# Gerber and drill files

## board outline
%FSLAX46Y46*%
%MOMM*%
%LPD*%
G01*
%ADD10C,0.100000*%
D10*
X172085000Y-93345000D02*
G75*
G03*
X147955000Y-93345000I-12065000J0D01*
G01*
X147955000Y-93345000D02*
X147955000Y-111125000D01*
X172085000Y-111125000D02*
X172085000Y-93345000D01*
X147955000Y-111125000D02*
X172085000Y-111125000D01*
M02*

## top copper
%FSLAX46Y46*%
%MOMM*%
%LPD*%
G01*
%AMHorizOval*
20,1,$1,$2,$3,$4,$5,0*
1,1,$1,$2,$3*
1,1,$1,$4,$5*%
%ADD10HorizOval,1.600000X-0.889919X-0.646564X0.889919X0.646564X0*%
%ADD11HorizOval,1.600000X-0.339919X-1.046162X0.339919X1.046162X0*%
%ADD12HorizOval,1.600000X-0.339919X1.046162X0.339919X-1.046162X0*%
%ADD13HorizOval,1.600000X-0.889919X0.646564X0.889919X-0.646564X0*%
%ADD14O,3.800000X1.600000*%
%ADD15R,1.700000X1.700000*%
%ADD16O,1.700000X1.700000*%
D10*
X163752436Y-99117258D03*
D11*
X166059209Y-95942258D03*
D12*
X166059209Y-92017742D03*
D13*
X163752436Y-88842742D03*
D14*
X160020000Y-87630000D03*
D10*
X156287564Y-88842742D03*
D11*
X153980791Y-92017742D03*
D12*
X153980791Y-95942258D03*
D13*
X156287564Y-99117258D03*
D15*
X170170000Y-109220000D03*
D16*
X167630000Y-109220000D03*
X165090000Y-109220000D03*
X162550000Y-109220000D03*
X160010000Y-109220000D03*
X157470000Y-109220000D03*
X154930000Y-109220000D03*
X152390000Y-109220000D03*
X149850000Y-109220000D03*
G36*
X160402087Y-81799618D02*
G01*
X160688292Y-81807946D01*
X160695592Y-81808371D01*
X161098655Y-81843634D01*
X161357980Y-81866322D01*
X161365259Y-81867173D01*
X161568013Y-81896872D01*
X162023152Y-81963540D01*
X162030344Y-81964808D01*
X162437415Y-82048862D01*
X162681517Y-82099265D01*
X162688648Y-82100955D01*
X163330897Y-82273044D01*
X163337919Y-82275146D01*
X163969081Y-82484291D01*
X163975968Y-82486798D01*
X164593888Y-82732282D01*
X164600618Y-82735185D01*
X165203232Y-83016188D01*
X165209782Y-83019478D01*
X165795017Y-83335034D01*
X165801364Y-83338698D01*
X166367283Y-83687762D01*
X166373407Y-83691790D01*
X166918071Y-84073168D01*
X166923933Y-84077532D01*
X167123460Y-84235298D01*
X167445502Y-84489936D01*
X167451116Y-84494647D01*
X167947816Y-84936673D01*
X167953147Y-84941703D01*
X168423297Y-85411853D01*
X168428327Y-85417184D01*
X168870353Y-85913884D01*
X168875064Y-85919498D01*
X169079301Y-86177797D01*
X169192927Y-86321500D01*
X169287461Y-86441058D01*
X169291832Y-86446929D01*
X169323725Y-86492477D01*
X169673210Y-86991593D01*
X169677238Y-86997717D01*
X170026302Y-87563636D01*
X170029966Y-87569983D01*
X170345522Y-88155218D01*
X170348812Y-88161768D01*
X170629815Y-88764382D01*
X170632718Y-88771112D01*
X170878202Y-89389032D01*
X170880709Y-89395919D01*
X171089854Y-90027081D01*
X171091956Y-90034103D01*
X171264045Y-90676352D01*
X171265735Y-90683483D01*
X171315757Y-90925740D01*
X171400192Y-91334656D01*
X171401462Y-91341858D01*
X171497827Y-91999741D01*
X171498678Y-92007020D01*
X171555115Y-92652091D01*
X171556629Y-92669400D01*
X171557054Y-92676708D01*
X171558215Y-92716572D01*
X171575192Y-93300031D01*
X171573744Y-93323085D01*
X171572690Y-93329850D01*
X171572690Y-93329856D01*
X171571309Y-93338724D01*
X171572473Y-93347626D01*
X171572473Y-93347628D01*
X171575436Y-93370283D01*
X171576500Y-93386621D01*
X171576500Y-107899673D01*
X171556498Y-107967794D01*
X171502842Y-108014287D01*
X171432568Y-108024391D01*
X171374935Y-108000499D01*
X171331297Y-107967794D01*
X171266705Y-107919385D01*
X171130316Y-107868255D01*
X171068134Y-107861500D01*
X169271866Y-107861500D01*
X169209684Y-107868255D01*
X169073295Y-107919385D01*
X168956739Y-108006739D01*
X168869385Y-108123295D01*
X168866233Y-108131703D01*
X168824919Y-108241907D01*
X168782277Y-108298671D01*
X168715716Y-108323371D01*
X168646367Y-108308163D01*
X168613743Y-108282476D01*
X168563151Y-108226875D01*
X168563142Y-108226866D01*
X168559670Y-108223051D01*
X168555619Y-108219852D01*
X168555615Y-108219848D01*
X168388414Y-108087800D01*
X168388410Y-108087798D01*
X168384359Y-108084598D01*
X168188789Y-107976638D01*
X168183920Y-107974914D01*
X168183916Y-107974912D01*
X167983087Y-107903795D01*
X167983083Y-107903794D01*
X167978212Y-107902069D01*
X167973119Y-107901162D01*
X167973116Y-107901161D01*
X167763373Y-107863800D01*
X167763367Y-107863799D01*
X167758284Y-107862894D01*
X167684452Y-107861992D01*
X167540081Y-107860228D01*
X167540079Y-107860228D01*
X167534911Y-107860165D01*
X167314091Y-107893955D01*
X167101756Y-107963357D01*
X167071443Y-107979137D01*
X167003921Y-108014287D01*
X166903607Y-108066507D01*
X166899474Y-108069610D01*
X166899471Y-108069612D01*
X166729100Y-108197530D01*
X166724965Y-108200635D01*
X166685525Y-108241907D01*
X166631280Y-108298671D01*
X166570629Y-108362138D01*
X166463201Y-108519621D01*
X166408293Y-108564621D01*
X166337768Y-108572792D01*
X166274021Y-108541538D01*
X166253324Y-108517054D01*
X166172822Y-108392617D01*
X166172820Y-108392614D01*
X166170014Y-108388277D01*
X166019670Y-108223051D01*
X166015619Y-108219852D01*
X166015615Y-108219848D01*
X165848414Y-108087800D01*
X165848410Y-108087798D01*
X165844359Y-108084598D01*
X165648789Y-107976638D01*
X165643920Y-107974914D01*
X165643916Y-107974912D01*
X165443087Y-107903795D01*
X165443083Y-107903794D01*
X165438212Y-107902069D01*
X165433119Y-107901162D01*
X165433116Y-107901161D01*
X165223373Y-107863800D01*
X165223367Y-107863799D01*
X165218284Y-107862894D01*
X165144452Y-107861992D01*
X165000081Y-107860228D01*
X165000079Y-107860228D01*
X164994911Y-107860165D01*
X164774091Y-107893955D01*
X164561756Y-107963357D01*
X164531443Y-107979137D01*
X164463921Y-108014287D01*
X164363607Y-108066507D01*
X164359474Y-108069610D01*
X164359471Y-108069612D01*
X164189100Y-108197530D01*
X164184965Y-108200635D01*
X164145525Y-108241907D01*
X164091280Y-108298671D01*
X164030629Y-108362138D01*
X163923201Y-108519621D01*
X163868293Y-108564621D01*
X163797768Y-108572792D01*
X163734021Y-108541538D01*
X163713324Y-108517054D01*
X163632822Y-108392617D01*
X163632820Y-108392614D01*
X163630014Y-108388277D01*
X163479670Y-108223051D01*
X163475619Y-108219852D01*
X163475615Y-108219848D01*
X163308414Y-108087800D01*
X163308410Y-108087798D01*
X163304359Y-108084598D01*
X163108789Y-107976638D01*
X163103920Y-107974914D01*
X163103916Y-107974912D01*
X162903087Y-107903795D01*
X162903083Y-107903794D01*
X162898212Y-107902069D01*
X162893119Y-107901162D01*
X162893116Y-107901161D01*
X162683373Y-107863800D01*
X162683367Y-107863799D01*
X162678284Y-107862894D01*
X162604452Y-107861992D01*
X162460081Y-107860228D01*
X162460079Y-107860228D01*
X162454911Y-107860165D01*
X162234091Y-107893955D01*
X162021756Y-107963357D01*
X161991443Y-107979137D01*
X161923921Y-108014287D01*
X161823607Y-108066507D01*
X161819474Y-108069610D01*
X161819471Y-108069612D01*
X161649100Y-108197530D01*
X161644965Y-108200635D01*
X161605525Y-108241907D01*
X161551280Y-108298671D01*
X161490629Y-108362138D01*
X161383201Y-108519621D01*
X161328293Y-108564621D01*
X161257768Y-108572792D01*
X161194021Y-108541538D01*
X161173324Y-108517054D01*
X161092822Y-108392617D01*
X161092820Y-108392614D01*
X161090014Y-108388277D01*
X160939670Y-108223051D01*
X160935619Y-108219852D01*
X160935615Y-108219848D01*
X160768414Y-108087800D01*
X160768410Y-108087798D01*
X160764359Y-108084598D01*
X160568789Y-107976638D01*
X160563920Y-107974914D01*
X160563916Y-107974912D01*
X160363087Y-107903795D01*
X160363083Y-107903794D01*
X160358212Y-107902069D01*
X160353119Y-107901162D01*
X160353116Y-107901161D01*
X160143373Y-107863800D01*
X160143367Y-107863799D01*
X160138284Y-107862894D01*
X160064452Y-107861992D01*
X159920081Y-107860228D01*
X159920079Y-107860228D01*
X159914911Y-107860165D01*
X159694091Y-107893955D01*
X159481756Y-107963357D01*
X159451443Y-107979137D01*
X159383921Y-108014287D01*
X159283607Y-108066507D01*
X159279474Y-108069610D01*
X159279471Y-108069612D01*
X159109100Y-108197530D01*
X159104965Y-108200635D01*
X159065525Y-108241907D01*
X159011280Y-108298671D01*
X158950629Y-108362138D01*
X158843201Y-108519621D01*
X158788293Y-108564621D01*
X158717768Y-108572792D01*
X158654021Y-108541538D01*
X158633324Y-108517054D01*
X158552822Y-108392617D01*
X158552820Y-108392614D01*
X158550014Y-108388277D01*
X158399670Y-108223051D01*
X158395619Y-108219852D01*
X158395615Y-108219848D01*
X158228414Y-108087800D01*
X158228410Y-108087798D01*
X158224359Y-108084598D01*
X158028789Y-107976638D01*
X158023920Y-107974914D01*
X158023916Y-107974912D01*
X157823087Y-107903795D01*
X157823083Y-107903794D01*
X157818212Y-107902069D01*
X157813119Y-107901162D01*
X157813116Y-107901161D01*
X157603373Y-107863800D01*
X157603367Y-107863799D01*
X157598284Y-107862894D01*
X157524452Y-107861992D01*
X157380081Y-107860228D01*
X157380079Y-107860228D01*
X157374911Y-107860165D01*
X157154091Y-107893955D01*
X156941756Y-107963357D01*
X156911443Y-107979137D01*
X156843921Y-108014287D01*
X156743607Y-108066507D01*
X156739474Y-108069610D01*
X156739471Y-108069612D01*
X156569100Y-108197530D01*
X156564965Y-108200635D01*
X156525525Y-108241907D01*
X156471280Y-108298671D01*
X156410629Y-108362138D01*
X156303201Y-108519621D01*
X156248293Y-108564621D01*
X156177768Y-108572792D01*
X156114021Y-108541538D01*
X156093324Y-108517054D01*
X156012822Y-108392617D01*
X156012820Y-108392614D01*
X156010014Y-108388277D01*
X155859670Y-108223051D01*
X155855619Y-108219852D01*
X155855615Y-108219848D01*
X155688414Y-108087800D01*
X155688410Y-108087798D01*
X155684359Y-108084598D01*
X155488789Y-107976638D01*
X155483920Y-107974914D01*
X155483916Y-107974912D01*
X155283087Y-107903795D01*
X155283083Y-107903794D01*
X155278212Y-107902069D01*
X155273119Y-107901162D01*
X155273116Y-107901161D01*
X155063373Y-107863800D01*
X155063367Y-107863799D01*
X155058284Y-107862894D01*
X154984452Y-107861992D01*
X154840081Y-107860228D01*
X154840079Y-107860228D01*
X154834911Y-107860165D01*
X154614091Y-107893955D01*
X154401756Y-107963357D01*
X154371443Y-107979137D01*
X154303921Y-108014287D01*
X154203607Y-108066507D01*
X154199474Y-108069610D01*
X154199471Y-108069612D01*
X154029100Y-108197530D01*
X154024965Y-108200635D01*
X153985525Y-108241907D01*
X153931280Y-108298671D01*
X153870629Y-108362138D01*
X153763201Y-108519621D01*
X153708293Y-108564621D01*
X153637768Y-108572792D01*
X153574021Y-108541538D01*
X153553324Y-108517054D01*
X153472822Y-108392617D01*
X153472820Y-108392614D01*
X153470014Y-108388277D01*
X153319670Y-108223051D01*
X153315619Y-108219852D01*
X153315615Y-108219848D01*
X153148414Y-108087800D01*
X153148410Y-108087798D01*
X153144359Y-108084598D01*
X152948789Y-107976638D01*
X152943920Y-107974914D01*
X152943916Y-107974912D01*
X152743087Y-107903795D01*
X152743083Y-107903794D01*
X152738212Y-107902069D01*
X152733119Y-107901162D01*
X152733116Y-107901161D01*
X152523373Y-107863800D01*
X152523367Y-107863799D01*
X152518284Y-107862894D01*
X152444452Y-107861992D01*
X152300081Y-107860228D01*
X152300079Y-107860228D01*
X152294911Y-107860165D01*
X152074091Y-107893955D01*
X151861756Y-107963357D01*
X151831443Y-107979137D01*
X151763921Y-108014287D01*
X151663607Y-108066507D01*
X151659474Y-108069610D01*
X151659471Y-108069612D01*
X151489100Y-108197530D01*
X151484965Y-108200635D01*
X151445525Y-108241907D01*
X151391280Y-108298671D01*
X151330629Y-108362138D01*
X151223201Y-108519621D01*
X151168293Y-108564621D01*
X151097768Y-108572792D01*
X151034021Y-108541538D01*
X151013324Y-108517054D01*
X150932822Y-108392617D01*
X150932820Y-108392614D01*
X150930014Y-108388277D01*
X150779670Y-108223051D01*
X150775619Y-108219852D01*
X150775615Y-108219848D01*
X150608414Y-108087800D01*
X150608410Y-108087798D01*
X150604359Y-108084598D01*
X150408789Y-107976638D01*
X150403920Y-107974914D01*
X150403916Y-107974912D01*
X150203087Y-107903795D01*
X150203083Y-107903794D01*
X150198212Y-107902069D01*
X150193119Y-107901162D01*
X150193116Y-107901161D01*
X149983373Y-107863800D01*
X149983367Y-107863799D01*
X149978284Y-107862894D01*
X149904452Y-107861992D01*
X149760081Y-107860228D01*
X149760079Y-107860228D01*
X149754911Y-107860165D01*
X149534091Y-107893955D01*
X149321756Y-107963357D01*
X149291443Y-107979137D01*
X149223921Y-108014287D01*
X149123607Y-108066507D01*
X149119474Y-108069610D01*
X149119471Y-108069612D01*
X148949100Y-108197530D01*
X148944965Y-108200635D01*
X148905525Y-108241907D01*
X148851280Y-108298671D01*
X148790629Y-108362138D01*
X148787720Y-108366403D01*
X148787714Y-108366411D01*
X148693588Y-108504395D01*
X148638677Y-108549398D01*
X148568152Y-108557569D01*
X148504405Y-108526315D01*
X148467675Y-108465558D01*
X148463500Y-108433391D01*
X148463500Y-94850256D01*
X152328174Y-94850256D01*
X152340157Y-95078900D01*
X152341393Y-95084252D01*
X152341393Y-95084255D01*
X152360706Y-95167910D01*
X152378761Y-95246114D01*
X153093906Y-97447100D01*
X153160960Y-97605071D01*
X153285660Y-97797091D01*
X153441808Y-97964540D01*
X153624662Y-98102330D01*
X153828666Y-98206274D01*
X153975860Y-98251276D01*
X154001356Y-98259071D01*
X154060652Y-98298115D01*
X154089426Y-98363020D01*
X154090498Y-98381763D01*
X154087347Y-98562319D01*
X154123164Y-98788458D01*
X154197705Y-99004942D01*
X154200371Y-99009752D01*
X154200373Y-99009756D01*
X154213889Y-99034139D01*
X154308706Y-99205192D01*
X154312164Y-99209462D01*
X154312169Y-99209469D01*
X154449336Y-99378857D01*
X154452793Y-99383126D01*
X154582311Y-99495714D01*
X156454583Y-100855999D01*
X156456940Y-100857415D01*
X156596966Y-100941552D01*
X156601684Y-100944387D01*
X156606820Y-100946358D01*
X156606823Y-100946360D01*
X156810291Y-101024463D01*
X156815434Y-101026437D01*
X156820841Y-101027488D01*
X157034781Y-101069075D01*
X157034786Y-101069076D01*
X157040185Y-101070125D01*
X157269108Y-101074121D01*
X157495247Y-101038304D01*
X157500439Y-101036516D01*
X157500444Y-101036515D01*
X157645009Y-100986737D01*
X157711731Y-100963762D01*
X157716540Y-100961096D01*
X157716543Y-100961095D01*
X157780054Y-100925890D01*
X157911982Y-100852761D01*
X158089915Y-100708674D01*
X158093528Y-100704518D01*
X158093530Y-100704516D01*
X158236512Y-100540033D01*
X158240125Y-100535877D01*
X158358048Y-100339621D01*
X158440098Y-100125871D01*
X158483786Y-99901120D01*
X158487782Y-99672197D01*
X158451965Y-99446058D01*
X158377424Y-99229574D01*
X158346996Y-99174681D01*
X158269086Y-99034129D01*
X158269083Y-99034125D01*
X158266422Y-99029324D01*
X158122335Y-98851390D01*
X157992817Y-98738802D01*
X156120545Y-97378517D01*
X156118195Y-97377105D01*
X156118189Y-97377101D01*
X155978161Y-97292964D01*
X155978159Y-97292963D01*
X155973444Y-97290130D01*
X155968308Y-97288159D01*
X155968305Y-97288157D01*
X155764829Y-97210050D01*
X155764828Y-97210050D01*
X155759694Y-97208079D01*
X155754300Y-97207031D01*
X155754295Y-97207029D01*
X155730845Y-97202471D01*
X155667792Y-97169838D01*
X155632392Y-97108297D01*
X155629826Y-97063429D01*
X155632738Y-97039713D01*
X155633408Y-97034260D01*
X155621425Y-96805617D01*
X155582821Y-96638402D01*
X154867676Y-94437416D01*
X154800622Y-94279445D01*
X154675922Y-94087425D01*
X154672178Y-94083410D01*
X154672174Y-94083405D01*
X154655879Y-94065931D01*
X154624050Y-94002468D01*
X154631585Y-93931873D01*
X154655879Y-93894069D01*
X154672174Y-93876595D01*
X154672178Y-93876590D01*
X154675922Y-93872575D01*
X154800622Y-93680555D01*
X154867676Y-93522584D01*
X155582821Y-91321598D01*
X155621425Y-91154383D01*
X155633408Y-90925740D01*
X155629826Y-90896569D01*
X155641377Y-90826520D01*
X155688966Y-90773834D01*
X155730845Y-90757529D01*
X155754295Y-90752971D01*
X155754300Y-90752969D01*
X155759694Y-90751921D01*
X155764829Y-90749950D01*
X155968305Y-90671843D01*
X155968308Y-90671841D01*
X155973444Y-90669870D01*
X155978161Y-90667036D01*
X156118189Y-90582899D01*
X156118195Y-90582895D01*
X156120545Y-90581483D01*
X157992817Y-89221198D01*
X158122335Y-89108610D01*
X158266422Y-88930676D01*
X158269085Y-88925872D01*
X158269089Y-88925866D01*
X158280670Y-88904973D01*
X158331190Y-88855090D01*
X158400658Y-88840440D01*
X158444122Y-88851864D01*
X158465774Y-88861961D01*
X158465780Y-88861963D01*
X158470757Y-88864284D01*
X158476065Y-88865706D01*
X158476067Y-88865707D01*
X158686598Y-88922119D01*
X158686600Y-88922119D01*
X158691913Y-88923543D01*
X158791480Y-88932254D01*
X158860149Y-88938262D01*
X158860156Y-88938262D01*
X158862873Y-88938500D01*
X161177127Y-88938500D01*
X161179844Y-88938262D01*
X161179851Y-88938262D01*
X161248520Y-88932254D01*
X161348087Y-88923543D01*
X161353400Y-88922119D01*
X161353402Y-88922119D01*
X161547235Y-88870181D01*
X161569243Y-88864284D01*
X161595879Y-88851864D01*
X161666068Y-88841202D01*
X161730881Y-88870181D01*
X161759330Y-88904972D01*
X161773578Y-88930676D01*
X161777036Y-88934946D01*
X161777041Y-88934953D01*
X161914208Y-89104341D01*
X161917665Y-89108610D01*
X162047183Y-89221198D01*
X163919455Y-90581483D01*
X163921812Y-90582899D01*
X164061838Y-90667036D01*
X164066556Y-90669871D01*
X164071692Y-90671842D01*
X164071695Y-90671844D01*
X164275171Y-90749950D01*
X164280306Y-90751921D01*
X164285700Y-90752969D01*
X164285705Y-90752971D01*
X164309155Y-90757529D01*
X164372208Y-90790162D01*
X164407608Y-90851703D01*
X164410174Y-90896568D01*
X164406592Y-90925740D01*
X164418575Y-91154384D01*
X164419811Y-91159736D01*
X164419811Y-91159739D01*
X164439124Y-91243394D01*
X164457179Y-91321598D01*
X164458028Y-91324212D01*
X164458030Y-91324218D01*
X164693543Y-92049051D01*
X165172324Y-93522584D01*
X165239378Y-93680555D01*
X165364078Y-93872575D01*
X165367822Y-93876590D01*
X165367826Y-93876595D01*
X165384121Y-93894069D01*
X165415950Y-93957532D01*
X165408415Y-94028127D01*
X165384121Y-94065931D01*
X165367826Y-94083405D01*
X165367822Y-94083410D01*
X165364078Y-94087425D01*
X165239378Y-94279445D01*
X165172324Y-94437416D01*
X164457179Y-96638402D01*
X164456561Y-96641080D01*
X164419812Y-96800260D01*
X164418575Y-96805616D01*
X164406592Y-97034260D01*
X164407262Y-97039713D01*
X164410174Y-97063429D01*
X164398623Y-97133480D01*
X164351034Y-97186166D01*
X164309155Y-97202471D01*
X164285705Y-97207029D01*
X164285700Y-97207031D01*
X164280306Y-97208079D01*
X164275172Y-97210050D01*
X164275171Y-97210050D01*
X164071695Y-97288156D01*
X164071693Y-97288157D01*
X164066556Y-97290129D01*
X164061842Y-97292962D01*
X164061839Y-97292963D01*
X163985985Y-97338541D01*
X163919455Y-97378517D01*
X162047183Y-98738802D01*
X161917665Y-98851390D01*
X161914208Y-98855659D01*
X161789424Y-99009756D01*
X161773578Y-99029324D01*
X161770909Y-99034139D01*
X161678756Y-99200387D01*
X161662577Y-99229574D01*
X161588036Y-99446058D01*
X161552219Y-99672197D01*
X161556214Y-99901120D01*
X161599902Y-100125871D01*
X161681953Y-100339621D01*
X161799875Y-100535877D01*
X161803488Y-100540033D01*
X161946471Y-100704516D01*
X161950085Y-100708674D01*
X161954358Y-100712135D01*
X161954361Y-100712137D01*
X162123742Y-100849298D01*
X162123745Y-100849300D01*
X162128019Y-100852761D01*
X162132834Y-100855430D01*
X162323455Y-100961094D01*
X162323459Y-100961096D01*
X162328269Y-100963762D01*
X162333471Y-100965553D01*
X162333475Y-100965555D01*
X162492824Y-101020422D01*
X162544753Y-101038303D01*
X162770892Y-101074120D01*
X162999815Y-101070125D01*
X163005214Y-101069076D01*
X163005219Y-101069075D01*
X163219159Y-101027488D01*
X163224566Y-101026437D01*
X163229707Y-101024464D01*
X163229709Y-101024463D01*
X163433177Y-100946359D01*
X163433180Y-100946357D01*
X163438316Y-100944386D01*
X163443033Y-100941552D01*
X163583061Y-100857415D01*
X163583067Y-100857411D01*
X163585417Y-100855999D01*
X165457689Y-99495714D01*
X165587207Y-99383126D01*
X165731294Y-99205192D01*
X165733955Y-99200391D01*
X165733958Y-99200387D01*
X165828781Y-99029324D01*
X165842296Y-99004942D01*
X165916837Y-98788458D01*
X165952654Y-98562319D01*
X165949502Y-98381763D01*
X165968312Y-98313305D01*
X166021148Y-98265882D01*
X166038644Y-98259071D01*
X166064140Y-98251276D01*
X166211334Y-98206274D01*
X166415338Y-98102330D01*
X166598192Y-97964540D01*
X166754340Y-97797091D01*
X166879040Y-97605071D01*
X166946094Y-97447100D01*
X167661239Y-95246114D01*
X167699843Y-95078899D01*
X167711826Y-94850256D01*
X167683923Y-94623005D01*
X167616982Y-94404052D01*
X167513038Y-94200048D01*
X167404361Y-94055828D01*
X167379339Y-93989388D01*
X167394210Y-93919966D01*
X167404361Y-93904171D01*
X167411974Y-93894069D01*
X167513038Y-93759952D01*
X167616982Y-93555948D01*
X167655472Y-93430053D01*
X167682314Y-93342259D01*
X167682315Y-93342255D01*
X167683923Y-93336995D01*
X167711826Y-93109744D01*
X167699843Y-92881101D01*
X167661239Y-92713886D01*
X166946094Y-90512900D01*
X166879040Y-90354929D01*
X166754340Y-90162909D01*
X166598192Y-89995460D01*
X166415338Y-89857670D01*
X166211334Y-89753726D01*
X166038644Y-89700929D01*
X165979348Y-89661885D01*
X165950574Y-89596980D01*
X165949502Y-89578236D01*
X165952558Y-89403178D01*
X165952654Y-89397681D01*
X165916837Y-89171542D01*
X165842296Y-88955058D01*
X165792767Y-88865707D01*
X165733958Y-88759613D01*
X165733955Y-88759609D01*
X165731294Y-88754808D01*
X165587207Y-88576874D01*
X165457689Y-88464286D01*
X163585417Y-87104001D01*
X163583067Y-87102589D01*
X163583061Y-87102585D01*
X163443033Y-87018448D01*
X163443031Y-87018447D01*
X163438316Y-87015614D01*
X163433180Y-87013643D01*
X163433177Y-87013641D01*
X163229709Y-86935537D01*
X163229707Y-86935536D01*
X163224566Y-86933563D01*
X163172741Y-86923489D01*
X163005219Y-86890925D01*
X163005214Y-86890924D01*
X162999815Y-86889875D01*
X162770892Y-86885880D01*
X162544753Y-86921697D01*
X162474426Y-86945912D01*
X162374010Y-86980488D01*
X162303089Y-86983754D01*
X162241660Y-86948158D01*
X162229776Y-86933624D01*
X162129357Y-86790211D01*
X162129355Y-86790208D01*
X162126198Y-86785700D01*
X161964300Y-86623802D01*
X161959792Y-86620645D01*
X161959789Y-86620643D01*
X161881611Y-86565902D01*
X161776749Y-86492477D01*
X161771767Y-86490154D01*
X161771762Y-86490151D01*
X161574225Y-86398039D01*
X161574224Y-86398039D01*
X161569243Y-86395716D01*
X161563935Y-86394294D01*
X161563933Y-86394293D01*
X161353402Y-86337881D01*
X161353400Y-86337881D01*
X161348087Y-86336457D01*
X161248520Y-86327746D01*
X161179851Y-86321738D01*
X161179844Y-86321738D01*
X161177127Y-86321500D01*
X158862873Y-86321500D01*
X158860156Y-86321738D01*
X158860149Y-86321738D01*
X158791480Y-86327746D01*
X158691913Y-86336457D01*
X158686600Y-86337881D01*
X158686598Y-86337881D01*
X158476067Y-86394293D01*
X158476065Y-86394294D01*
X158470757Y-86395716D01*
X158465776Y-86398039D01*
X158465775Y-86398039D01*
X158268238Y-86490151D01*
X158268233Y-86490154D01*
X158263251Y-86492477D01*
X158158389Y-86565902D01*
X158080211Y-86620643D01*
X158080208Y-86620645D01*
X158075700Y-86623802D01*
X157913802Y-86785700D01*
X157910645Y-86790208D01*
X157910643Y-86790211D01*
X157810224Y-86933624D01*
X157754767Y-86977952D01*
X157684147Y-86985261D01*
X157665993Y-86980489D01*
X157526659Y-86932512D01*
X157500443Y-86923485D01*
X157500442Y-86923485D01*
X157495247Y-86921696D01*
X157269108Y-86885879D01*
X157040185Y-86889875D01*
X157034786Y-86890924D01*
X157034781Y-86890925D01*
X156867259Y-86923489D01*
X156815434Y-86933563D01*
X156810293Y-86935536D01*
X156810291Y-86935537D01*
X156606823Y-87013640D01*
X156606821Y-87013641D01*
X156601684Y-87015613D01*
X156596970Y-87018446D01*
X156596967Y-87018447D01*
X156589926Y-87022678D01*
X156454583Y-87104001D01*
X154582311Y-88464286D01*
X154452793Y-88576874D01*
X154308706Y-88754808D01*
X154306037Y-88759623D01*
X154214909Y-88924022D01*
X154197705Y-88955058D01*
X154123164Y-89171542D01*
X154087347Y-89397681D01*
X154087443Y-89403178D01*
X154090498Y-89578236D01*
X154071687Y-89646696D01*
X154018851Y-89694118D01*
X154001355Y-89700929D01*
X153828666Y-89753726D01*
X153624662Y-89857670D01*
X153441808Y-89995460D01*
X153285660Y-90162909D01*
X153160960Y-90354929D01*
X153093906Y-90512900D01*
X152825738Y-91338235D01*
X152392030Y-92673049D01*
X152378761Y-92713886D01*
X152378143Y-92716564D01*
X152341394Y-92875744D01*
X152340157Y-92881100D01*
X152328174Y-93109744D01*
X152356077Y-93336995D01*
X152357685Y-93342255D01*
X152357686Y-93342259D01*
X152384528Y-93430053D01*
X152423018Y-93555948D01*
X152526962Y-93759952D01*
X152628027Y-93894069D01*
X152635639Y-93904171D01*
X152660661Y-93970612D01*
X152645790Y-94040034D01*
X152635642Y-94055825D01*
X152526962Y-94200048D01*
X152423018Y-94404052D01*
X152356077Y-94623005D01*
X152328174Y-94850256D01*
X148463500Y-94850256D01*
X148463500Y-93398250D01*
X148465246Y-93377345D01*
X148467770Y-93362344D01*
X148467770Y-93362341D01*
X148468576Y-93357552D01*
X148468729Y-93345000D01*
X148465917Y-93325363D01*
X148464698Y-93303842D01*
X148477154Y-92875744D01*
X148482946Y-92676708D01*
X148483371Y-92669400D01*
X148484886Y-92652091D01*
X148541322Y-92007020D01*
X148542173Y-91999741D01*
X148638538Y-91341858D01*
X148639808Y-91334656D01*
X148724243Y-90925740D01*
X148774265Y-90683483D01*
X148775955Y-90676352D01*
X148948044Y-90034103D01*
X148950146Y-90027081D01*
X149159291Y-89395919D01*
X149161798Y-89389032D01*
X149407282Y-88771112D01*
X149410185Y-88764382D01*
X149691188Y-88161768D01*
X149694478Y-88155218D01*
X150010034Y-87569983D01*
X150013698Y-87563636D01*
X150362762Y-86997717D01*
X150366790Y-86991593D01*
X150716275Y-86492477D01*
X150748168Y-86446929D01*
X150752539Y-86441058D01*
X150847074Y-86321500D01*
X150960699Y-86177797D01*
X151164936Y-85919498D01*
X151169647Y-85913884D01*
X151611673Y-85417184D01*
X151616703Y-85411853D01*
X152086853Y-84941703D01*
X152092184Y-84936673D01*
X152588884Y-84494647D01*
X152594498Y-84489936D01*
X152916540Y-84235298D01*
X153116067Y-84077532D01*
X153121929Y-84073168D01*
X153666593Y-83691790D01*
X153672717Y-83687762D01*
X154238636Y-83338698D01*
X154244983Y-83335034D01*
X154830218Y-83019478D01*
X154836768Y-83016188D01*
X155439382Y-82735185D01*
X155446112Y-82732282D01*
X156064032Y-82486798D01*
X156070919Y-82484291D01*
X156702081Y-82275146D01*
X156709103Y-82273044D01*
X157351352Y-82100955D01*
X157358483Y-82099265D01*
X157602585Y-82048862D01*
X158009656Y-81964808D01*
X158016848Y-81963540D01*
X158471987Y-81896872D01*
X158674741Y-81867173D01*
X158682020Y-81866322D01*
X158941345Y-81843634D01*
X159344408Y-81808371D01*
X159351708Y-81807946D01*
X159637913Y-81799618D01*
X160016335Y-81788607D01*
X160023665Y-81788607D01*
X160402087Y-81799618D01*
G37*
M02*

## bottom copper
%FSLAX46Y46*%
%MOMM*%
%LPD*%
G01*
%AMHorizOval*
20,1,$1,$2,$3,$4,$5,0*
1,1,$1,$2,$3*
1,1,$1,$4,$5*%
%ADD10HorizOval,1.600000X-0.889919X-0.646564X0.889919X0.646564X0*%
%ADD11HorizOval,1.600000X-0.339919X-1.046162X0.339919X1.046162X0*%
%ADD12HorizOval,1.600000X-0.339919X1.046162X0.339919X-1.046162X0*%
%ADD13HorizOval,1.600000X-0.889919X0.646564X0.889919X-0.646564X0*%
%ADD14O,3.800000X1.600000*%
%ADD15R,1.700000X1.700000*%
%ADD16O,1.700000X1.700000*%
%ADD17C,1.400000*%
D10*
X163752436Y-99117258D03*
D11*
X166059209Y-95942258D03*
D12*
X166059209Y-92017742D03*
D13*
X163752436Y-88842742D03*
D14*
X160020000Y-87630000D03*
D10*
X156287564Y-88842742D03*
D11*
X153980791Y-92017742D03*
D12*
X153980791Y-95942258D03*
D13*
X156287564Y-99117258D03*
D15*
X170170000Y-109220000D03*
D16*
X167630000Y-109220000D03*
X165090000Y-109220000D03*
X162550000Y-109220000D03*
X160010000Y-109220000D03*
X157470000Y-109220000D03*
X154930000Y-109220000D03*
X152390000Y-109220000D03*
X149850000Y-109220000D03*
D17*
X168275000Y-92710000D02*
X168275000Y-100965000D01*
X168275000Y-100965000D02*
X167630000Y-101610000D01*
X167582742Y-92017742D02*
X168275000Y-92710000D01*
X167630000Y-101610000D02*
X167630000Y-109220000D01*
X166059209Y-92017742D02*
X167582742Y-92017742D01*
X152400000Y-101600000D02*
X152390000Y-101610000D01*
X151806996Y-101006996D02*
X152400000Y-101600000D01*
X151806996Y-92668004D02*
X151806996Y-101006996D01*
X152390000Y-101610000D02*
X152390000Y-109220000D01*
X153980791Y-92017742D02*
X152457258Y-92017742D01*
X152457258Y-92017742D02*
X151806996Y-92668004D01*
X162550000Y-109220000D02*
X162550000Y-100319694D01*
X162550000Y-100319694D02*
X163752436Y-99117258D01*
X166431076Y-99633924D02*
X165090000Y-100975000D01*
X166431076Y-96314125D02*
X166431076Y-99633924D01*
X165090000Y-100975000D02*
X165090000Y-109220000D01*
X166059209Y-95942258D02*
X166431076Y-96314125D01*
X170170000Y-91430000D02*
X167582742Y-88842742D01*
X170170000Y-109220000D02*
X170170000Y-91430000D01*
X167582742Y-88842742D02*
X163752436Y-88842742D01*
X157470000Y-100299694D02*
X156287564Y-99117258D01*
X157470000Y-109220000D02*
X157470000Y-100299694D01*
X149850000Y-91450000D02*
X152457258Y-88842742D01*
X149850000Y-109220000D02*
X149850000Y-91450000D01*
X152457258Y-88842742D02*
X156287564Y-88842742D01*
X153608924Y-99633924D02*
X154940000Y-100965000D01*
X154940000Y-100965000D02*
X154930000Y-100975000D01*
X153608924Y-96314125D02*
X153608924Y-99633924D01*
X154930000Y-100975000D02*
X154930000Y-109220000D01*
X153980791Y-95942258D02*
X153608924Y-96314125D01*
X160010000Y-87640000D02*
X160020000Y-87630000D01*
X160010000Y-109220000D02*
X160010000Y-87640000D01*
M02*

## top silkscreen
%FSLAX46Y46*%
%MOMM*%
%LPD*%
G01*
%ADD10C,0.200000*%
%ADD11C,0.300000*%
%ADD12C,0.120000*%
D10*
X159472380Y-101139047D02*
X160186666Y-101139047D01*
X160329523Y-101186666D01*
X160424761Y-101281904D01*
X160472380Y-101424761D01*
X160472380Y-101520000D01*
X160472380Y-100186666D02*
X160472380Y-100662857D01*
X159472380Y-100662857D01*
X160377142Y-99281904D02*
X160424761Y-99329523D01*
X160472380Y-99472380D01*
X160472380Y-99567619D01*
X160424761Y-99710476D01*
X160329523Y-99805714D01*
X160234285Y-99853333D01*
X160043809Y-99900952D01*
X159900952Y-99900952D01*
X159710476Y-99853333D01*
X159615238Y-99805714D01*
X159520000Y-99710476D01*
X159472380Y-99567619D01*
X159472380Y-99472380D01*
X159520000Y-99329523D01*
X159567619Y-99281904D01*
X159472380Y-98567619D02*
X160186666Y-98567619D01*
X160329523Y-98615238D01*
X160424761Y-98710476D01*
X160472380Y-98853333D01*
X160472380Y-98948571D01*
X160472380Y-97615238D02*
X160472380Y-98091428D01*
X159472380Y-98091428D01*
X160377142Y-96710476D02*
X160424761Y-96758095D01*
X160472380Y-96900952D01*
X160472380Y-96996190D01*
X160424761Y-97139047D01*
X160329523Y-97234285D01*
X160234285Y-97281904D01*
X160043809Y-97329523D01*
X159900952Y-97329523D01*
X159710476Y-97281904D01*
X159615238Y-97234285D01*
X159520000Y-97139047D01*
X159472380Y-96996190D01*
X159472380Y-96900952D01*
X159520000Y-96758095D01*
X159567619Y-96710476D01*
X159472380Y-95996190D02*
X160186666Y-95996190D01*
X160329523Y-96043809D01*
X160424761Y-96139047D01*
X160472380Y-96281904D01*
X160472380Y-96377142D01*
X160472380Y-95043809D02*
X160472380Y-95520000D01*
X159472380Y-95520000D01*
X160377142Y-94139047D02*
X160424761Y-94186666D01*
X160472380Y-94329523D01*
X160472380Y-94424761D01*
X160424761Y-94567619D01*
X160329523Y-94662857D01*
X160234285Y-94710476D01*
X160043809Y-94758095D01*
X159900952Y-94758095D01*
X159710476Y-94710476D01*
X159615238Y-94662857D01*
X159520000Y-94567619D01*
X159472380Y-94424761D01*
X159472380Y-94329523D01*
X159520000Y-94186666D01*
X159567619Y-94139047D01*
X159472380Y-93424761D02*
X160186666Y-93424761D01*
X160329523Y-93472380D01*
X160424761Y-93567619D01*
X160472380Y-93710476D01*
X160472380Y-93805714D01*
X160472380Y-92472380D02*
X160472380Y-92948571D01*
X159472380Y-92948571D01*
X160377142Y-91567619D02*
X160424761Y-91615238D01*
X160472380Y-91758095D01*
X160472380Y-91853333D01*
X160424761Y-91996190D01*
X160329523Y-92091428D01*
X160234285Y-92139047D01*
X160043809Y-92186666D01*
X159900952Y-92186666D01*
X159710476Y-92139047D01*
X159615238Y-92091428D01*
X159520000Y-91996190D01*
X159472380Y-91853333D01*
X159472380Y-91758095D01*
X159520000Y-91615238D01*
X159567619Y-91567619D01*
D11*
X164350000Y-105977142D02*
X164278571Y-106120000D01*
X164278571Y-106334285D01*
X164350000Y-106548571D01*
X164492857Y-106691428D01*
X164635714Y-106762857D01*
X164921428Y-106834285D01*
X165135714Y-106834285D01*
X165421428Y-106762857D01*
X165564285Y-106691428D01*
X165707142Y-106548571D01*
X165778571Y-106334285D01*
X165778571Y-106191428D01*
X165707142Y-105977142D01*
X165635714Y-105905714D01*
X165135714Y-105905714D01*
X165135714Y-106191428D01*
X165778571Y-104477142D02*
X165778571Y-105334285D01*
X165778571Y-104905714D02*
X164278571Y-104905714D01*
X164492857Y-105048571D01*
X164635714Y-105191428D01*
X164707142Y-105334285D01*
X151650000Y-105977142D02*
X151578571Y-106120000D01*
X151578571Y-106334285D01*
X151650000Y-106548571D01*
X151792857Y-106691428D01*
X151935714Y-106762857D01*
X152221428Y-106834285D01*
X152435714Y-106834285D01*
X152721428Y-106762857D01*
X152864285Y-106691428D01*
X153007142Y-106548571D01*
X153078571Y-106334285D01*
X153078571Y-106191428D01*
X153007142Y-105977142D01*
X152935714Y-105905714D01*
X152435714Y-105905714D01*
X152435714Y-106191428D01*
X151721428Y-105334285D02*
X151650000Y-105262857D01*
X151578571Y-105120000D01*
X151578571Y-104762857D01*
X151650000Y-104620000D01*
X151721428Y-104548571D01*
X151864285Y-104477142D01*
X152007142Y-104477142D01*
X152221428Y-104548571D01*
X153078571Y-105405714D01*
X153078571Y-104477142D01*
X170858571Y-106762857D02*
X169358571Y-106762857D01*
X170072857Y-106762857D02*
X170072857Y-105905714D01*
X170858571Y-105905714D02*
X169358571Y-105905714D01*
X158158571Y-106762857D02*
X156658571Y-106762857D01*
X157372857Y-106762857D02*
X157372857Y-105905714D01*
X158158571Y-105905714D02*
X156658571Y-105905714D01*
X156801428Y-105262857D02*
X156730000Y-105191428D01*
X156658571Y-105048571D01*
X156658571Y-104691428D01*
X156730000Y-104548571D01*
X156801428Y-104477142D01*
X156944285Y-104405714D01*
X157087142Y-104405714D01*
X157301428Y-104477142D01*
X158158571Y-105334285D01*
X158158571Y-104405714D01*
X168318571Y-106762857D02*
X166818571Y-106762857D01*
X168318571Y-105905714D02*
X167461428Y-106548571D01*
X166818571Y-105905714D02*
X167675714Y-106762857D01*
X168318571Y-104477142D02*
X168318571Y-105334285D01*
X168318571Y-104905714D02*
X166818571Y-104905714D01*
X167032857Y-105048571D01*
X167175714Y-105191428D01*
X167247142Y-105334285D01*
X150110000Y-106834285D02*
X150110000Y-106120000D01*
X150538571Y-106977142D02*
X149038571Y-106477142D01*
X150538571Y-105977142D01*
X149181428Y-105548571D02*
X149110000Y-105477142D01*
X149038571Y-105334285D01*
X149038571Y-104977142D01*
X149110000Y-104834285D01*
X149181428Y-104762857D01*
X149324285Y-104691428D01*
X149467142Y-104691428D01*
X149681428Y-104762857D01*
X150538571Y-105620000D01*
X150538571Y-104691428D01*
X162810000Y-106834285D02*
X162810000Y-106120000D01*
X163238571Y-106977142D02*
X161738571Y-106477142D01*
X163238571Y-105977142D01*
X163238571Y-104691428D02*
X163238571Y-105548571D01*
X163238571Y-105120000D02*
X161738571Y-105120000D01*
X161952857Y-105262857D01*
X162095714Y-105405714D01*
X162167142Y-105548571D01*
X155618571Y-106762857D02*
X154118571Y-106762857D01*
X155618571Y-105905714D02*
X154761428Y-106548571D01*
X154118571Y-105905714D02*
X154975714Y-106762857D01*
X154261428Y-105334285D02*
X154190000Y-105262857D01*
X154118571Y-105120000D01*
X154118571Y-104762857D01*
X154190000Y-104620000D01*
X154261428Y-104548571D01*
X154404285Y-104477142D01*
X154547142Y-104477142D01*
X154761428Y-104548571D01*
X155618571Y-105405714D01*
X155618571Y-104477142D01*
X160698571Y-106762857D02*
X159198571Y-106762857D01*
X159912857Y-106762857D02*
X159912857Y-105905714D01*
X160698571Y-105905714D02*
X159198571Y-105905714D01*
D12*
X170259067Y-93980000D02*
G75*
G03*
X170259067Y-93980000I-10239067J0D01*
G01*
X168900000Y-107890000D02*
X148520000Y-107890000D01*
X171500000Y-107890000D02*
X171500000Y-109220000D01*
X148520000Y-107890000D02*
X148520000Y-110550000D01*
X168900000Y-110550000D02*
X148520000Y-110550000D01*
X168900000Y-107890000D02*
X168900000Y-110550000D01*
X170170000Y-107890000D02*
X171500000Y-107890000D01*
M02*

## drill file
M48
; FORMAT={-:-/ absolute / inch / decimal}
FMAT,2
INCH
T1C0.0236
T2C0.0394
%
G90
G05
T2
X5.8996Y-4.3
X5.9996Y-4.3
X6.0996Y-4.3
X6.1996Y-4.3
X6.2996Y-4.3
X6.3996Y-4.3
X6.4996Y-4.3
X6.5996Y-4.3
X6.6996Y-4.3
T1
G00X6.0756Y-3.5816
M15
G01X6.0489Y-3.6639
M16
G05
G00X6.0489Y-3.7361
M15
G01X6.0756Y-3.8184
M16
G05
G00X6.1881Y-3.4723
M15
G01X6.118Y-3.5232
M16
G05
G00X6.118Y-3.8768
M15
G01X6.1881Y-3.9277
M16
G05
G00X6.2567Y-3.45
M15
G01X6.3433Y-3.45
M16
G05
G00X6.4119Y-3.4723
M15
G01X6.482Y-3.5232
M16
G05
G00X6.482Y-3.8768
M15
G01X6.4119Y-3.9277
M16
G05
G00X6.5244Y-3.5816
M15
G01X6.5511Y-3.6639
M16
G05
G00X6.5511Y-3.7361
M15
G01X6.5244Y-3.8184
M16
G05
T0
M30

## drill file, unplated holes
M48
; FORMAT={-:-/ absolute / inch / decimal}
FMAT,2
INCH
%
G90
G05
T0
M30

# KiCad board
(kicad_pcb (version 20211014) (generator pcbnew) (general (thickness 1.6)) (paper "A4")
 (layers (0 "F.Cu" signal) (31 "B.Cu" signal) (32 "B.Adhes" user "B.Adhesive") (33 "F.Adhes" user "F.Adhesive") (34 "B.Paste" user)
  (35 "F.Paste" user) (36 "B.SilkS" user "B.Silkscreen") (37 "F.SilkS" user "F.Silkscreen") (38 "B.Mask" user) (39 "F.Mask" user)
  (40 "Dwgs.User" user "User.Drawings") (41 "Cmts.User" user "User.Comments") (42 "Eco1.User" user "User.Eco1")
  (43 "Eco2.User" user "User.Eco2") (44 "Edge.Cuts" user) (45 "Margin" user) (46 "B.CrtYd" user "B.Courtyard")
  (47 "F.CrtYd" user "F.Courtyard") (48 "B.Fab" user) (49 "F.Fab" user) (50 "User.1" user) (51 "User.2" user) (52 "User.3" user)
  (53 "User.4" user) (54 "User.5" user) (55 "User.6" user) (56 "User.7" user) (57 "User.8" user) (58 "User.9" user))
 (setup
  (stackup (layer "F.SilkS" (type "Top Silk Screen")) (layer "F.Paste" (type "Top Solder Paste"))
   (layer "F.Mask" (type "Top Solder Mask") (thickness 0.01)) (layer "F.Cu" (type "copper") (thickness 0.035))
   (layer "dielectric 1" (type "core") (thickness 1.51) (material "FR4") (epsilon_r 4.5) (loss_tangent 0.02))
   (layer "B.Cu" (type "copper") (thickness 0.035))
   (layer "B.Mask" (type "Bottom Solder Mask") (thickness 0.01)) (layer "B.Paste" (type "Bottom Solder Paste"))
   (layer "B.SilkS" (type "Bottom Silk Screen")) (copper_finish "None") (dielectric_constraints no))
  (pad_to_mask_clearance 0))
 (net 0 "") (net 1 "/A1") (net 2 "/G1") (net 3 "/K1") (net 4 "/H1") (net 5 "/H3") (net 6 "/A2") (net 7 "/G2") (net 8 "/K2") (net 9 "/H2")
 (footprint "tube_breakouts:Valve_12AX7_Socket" (layer "F.Cu") (at 160.02 93.98)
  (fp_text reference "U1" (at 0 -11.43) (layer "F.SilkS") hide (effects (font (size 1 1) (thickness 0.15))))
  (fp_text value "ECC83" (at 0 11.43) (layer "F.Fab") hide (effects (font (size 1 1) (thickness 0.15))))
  (fp_circle (center 0 0) (end 10.16 1.27) (layer "F.SilkS") (width 0.12) (fill none))
  (pad "1" thru_hole oval (at 3.732436 5.137258 306) (size 1.6 3.8) (drill oval 0.6 2.8) (layers *.Cu *.Mask) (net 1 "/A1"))
  (pad "2" thru_hole oval (at 6.039209 1.962258 342) (size 1.6 3.8) (drill oval 0.6 2.8) (layers *.Cu *.Mask) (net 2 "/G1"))
  (pad "3" thru_hole oval (at 6.039209 -1.962258 18) (size 1.6 3.8) (drill oval 0.6 2.8) (layers *.Cu *.Mask) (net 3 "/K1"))
  (pad "4" thru_hole oval (at 3.732436 -5.137258 54) (size 1.6 3.8) (drill oval 0.6 2.8) (layers *.Cu *.Mask) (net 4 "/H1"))
  (pad "5" thru_hole oval (at 0 -6.35 90) (size 1.6 3.8) (drill oval 0.6 2.8) (layers *.Cu *.Mask) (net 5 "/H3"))
  (pad "6" thru_hole oval (at -3.732436 -5.137258 306) (size 1.6 3.8) (drill oval 0.6 2.8) (layers *.Cu *.Mask) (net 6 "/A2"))
  (pad "7" thru_hole oval (at -6.039209 -1.962258 342) (size 1.6 3.8) (drill oval 0.6 2.8) (layers *.Cu *.Mask) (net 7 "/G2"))
  (pad "8" thru_hole oval (at -6.039209 1.962258 18) (size 1.6 3.8) (drill oval 0.6 2.8) (layers *.Cu *.Mask) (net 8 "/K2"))
  (pad "9" thru_hole oval (at -3.732436 5.137258 54) (size 1.6 3.8) (drill oval 0.6 2.8) (layers *.Cu *.Mask) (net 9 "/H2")))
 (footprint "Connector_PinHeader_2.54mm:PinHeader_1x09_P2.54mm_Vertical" (layer "F.Cu") (at 170.17 109.22 -90)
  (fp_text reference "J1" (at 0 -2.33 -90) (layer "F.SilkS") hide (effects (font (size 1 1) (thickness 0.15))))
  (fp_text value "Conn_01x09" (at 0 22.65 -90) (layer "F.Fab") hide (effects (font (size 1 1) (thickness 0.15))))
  (fp_line (start -1.33 1.27) (end -1.33 21.65) (layer "F.SilkS") (width 0.12))
  (fp_line (start -1.33 -1.33) (end 0 -1.33) (layer "F.SilkS") (width 0.12))
  (fp_line (start -1.33 21.65) (end 1.33 21.65) (layer "F.SilkS") (width 0.12))
  (fp_line (start 1.33 1.27) (end 1.33 21.65) (layer "F.SilkS") (width 0.12))
  (fp_line (start -1.33 1.27) (end 1.33 1.27) (layer "F.SilkS") (width 0.12))
  (fp_line (start -1.33 0) (end -1.33 -1.33) (layer "F.SilkS") (width 0.12))
  (pad "1" thru_hole rect (at 0 0 270) (size 1.7 1.7) (drill 1) (layers *.Cu *.Mask) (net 4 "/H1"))
  (pad "2" thru_hole oval (at 0 2.54 270) (size 1.7 1.7) (drill 1) (layers *.Cu *.Mask) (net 3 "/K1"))
  (pad "3" thru_hole oval (at 0 5.08 270) (size 1.7 1.7) (drill 1) (layers *.Cu *.Mask) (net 2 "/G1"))
  (pad "4" thru_hole oval (at 0 7.62 270) (size 1.7 1.7) (drill 1) (layers *.Cu *.Mask) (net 1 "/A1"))
  (pad "5" thru_hole oval (at 0 10.16 270) (size 1.7 1.7) (drill 1) (layers *.Cu *.Mask) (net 5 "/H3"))
  (pad "6" thru_hole oval (at 0 12.7 270) (size 1.7 1.7) (drill 1) (layers *.Cu *.Mask) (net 9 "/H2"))
  (pad "7" thru_hole oval (at 0 15.24 270) (size 1.7 1.7) (drill 1) (layers *.Cu *.Mask) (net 8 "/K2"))
  (pad "8" thru_hole oval (at 0 17.78 270) (size 1.7 1.7) (drill 1) (layers *.Cu *.Mask) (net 7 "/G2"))
  (pad "9" thru_hole oval (at 0 20.32 270) (size 1.7 1.7) (drill 1) (layers *.Cu *.Mask) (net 6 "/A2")))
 (gr_arc (start 147.955 93.345) (mid 160.02 81.28) (end 172.085 93.345) (layer "Edge.Cuts") (width 0.1))
 (gr_line (start 147.955 93.345) (end 147.955 111.125) (layer "Edge.Cuts") (width 0.1))
 (gr_line (start 172.085 111.125) (end 172.085 93.345) (layer "Edge.Cuts") (width 0.1))
 (gr_line (start 147.955 111.125) (end 172.085 111.125) (layer "Edge.Cuts") (width 0.1))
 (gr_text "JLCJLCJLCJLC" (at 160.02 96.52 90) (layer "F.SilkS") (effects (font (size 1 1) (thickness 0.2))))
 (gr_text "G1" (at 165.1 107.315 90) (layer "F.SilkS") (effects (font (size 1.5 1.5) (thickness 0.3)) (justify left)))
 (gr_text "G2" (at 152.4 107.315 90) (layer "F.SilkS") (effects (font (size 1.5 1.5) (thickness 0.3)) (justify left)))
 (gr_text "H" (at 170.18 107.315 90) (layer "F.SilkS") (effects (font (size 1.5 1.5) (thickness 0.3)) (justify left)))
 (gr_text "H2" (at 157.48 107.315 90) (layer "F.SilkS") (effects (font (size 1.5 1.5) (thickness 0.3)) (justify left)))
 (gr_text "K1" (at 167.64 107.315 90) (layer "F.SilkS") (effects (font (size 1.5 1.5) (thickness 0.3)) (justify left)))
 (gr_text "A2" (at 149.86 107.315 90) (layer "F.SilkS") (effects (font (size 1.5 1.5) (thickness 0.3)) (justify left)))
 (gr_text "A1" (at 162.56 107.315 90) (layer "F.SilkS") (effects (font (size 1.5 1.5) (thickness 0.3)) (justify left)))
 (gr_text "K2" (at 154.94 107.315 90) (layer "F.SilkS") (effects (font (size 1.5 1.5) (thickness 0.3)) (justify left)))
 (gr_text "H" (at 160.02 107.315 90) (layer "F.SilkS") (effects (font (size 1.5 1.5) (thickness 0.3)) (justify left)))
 (segment (start 162.55 109.22) (end 162.55 100.319694) (width 1.4) (layer "B.Cu") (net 1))
 (segment (start 162.55 100.319694) (end 163.752436 99.117258) (width 1.4) (layer "B.Cu") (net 1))
 (segment (start 166.431076 99.633924) (end 165.09 100.975) (width 1.4) (layer "B.Cu") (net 2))
 (segment (start 166.431076 96.314125) (end 166.431076 99.633924) (width 1.4) (layer "B.Cu") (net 2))
 (segment (start 165.09 100.975) (end 165.09 109.22) (width 1.4) (layer "B.Cu") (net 2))
 (segment (start 166.059209 95.942258) (end 166.431076 96.314125) (width 1.4) (layer "B.Cu") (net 2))
 (segment (start 168.275 92.71) (end 168.275 100.965) (width 1.4) (layer "B.Cu") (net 3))
 (segment (start 167.582742 92.017742) (end 168.275 92.71) (width 1.4) (layer "B.Cu") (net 3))
 (segment (start 168.275 100.965) (end 167.63 101.61) (width 1.4) (layer "B.Cu") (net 3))
 (segment (start 166.059209 92.017742) (end 167.582742 92.017742) (width 1.4) (layer "B.Cu") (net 3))
 (segment (start 167.63 101.61) (end 167.63 109.22) (width 1.4) (layer "B.Cu") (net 3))
 (segment (start 170.17 91.43) (end 167.582742 88.842742) (width 1.4) (layer "B.Cu") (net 4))
 (segment (start 170.17 109.22) (end 170.17 91.43) (width 1.4) (layer "B.Cu") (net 4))
 (segment (start 167.582742 88.842742) (end 163.752436 88.842742) (width 1.4) (layer "B.Cu") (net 4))
 (segment (start 157.47 100.299694) (end 156.287564 99.117258) (width 1.4) (layer "B.Cu") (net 9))
 (segment (start 157.47 109.22) (end 157.47 100.299694) (width 1.4) (layer "B.Cu") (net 9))
 (segment (start 149.85 91.45) (end 152.457258 88.842742) (width 1.4) (layer "B.Cu") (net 6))
 (segment (start 149.85 109.22) (end 149.85 91.45) (width 1.4) (layer "B.Cu") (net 6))
 (segment (start 152.457258 88.842742) (end 156.287564 88.842742) (width 1.4) (layer "B.Cu") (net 6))
 (segment (start 153.980791 92.017742) (end 152.457258 92.017742) (width 1.4) (layer "B.Cu") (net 7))
 (segment (start 151.806996 92.668004) (end 151.806996 101.006996) (width 1.4) (layer "B.Cu") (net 7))
 (segment (start 151.806996 101.006996) (end 152.4 101.6) (width 1.4) (layer "B.Cu") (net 7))
 (segment (start 152.39 101.61) (end 152.39 109.22) (width 1.4) (layer "B.Cu") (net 7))
 (segment (start 152.4 101.6) (end 152.39 101.61) (width 1.4) (layer "B.Cu") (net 7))
 (segment (start 152.457258 92.017742) (end 151.806996 92.668004) (width 1.4) (layer "B.Cu") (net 7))
 (segment (start 153.608924 99.633924) (end 154.94 100.965) (width 1.4) (layer "B.Cu") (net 8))
 (segment (start 154.94 100.965) (end 154.93 100.975) (width 1.4) (layer "B.Cu") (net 8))
 (segment (start 153.608924 96.314125) (end 153.608924 99.633924) (width 1.4) (layer "B.Cu") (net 8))
 (segment (start 154.93 100.975) (end 154.93 109.22) (width 1.4) (layer "B.Cu") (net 8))
 (segment (start 153.980791 95.942258) (end 153.608924 96.314125) (width 1.4) (layer "B.Cu") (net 8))
 (segment (start 160.01 87.64) (end 160.02 87.63) (width 1.4) (layer "B.Cu") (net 5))
 (segment (start 160.01 109.22) (end 160.01 87.64) (width 1.4) (layer "B.Cu") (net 5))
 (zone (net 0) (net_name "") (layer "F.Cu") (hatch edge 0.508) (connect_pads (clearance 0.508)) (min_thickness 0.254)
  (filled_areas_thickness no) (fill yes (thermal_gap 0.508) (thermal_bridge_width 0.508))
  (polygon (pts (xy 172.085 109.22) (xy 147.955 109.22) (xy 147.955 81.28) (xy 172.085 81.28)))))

